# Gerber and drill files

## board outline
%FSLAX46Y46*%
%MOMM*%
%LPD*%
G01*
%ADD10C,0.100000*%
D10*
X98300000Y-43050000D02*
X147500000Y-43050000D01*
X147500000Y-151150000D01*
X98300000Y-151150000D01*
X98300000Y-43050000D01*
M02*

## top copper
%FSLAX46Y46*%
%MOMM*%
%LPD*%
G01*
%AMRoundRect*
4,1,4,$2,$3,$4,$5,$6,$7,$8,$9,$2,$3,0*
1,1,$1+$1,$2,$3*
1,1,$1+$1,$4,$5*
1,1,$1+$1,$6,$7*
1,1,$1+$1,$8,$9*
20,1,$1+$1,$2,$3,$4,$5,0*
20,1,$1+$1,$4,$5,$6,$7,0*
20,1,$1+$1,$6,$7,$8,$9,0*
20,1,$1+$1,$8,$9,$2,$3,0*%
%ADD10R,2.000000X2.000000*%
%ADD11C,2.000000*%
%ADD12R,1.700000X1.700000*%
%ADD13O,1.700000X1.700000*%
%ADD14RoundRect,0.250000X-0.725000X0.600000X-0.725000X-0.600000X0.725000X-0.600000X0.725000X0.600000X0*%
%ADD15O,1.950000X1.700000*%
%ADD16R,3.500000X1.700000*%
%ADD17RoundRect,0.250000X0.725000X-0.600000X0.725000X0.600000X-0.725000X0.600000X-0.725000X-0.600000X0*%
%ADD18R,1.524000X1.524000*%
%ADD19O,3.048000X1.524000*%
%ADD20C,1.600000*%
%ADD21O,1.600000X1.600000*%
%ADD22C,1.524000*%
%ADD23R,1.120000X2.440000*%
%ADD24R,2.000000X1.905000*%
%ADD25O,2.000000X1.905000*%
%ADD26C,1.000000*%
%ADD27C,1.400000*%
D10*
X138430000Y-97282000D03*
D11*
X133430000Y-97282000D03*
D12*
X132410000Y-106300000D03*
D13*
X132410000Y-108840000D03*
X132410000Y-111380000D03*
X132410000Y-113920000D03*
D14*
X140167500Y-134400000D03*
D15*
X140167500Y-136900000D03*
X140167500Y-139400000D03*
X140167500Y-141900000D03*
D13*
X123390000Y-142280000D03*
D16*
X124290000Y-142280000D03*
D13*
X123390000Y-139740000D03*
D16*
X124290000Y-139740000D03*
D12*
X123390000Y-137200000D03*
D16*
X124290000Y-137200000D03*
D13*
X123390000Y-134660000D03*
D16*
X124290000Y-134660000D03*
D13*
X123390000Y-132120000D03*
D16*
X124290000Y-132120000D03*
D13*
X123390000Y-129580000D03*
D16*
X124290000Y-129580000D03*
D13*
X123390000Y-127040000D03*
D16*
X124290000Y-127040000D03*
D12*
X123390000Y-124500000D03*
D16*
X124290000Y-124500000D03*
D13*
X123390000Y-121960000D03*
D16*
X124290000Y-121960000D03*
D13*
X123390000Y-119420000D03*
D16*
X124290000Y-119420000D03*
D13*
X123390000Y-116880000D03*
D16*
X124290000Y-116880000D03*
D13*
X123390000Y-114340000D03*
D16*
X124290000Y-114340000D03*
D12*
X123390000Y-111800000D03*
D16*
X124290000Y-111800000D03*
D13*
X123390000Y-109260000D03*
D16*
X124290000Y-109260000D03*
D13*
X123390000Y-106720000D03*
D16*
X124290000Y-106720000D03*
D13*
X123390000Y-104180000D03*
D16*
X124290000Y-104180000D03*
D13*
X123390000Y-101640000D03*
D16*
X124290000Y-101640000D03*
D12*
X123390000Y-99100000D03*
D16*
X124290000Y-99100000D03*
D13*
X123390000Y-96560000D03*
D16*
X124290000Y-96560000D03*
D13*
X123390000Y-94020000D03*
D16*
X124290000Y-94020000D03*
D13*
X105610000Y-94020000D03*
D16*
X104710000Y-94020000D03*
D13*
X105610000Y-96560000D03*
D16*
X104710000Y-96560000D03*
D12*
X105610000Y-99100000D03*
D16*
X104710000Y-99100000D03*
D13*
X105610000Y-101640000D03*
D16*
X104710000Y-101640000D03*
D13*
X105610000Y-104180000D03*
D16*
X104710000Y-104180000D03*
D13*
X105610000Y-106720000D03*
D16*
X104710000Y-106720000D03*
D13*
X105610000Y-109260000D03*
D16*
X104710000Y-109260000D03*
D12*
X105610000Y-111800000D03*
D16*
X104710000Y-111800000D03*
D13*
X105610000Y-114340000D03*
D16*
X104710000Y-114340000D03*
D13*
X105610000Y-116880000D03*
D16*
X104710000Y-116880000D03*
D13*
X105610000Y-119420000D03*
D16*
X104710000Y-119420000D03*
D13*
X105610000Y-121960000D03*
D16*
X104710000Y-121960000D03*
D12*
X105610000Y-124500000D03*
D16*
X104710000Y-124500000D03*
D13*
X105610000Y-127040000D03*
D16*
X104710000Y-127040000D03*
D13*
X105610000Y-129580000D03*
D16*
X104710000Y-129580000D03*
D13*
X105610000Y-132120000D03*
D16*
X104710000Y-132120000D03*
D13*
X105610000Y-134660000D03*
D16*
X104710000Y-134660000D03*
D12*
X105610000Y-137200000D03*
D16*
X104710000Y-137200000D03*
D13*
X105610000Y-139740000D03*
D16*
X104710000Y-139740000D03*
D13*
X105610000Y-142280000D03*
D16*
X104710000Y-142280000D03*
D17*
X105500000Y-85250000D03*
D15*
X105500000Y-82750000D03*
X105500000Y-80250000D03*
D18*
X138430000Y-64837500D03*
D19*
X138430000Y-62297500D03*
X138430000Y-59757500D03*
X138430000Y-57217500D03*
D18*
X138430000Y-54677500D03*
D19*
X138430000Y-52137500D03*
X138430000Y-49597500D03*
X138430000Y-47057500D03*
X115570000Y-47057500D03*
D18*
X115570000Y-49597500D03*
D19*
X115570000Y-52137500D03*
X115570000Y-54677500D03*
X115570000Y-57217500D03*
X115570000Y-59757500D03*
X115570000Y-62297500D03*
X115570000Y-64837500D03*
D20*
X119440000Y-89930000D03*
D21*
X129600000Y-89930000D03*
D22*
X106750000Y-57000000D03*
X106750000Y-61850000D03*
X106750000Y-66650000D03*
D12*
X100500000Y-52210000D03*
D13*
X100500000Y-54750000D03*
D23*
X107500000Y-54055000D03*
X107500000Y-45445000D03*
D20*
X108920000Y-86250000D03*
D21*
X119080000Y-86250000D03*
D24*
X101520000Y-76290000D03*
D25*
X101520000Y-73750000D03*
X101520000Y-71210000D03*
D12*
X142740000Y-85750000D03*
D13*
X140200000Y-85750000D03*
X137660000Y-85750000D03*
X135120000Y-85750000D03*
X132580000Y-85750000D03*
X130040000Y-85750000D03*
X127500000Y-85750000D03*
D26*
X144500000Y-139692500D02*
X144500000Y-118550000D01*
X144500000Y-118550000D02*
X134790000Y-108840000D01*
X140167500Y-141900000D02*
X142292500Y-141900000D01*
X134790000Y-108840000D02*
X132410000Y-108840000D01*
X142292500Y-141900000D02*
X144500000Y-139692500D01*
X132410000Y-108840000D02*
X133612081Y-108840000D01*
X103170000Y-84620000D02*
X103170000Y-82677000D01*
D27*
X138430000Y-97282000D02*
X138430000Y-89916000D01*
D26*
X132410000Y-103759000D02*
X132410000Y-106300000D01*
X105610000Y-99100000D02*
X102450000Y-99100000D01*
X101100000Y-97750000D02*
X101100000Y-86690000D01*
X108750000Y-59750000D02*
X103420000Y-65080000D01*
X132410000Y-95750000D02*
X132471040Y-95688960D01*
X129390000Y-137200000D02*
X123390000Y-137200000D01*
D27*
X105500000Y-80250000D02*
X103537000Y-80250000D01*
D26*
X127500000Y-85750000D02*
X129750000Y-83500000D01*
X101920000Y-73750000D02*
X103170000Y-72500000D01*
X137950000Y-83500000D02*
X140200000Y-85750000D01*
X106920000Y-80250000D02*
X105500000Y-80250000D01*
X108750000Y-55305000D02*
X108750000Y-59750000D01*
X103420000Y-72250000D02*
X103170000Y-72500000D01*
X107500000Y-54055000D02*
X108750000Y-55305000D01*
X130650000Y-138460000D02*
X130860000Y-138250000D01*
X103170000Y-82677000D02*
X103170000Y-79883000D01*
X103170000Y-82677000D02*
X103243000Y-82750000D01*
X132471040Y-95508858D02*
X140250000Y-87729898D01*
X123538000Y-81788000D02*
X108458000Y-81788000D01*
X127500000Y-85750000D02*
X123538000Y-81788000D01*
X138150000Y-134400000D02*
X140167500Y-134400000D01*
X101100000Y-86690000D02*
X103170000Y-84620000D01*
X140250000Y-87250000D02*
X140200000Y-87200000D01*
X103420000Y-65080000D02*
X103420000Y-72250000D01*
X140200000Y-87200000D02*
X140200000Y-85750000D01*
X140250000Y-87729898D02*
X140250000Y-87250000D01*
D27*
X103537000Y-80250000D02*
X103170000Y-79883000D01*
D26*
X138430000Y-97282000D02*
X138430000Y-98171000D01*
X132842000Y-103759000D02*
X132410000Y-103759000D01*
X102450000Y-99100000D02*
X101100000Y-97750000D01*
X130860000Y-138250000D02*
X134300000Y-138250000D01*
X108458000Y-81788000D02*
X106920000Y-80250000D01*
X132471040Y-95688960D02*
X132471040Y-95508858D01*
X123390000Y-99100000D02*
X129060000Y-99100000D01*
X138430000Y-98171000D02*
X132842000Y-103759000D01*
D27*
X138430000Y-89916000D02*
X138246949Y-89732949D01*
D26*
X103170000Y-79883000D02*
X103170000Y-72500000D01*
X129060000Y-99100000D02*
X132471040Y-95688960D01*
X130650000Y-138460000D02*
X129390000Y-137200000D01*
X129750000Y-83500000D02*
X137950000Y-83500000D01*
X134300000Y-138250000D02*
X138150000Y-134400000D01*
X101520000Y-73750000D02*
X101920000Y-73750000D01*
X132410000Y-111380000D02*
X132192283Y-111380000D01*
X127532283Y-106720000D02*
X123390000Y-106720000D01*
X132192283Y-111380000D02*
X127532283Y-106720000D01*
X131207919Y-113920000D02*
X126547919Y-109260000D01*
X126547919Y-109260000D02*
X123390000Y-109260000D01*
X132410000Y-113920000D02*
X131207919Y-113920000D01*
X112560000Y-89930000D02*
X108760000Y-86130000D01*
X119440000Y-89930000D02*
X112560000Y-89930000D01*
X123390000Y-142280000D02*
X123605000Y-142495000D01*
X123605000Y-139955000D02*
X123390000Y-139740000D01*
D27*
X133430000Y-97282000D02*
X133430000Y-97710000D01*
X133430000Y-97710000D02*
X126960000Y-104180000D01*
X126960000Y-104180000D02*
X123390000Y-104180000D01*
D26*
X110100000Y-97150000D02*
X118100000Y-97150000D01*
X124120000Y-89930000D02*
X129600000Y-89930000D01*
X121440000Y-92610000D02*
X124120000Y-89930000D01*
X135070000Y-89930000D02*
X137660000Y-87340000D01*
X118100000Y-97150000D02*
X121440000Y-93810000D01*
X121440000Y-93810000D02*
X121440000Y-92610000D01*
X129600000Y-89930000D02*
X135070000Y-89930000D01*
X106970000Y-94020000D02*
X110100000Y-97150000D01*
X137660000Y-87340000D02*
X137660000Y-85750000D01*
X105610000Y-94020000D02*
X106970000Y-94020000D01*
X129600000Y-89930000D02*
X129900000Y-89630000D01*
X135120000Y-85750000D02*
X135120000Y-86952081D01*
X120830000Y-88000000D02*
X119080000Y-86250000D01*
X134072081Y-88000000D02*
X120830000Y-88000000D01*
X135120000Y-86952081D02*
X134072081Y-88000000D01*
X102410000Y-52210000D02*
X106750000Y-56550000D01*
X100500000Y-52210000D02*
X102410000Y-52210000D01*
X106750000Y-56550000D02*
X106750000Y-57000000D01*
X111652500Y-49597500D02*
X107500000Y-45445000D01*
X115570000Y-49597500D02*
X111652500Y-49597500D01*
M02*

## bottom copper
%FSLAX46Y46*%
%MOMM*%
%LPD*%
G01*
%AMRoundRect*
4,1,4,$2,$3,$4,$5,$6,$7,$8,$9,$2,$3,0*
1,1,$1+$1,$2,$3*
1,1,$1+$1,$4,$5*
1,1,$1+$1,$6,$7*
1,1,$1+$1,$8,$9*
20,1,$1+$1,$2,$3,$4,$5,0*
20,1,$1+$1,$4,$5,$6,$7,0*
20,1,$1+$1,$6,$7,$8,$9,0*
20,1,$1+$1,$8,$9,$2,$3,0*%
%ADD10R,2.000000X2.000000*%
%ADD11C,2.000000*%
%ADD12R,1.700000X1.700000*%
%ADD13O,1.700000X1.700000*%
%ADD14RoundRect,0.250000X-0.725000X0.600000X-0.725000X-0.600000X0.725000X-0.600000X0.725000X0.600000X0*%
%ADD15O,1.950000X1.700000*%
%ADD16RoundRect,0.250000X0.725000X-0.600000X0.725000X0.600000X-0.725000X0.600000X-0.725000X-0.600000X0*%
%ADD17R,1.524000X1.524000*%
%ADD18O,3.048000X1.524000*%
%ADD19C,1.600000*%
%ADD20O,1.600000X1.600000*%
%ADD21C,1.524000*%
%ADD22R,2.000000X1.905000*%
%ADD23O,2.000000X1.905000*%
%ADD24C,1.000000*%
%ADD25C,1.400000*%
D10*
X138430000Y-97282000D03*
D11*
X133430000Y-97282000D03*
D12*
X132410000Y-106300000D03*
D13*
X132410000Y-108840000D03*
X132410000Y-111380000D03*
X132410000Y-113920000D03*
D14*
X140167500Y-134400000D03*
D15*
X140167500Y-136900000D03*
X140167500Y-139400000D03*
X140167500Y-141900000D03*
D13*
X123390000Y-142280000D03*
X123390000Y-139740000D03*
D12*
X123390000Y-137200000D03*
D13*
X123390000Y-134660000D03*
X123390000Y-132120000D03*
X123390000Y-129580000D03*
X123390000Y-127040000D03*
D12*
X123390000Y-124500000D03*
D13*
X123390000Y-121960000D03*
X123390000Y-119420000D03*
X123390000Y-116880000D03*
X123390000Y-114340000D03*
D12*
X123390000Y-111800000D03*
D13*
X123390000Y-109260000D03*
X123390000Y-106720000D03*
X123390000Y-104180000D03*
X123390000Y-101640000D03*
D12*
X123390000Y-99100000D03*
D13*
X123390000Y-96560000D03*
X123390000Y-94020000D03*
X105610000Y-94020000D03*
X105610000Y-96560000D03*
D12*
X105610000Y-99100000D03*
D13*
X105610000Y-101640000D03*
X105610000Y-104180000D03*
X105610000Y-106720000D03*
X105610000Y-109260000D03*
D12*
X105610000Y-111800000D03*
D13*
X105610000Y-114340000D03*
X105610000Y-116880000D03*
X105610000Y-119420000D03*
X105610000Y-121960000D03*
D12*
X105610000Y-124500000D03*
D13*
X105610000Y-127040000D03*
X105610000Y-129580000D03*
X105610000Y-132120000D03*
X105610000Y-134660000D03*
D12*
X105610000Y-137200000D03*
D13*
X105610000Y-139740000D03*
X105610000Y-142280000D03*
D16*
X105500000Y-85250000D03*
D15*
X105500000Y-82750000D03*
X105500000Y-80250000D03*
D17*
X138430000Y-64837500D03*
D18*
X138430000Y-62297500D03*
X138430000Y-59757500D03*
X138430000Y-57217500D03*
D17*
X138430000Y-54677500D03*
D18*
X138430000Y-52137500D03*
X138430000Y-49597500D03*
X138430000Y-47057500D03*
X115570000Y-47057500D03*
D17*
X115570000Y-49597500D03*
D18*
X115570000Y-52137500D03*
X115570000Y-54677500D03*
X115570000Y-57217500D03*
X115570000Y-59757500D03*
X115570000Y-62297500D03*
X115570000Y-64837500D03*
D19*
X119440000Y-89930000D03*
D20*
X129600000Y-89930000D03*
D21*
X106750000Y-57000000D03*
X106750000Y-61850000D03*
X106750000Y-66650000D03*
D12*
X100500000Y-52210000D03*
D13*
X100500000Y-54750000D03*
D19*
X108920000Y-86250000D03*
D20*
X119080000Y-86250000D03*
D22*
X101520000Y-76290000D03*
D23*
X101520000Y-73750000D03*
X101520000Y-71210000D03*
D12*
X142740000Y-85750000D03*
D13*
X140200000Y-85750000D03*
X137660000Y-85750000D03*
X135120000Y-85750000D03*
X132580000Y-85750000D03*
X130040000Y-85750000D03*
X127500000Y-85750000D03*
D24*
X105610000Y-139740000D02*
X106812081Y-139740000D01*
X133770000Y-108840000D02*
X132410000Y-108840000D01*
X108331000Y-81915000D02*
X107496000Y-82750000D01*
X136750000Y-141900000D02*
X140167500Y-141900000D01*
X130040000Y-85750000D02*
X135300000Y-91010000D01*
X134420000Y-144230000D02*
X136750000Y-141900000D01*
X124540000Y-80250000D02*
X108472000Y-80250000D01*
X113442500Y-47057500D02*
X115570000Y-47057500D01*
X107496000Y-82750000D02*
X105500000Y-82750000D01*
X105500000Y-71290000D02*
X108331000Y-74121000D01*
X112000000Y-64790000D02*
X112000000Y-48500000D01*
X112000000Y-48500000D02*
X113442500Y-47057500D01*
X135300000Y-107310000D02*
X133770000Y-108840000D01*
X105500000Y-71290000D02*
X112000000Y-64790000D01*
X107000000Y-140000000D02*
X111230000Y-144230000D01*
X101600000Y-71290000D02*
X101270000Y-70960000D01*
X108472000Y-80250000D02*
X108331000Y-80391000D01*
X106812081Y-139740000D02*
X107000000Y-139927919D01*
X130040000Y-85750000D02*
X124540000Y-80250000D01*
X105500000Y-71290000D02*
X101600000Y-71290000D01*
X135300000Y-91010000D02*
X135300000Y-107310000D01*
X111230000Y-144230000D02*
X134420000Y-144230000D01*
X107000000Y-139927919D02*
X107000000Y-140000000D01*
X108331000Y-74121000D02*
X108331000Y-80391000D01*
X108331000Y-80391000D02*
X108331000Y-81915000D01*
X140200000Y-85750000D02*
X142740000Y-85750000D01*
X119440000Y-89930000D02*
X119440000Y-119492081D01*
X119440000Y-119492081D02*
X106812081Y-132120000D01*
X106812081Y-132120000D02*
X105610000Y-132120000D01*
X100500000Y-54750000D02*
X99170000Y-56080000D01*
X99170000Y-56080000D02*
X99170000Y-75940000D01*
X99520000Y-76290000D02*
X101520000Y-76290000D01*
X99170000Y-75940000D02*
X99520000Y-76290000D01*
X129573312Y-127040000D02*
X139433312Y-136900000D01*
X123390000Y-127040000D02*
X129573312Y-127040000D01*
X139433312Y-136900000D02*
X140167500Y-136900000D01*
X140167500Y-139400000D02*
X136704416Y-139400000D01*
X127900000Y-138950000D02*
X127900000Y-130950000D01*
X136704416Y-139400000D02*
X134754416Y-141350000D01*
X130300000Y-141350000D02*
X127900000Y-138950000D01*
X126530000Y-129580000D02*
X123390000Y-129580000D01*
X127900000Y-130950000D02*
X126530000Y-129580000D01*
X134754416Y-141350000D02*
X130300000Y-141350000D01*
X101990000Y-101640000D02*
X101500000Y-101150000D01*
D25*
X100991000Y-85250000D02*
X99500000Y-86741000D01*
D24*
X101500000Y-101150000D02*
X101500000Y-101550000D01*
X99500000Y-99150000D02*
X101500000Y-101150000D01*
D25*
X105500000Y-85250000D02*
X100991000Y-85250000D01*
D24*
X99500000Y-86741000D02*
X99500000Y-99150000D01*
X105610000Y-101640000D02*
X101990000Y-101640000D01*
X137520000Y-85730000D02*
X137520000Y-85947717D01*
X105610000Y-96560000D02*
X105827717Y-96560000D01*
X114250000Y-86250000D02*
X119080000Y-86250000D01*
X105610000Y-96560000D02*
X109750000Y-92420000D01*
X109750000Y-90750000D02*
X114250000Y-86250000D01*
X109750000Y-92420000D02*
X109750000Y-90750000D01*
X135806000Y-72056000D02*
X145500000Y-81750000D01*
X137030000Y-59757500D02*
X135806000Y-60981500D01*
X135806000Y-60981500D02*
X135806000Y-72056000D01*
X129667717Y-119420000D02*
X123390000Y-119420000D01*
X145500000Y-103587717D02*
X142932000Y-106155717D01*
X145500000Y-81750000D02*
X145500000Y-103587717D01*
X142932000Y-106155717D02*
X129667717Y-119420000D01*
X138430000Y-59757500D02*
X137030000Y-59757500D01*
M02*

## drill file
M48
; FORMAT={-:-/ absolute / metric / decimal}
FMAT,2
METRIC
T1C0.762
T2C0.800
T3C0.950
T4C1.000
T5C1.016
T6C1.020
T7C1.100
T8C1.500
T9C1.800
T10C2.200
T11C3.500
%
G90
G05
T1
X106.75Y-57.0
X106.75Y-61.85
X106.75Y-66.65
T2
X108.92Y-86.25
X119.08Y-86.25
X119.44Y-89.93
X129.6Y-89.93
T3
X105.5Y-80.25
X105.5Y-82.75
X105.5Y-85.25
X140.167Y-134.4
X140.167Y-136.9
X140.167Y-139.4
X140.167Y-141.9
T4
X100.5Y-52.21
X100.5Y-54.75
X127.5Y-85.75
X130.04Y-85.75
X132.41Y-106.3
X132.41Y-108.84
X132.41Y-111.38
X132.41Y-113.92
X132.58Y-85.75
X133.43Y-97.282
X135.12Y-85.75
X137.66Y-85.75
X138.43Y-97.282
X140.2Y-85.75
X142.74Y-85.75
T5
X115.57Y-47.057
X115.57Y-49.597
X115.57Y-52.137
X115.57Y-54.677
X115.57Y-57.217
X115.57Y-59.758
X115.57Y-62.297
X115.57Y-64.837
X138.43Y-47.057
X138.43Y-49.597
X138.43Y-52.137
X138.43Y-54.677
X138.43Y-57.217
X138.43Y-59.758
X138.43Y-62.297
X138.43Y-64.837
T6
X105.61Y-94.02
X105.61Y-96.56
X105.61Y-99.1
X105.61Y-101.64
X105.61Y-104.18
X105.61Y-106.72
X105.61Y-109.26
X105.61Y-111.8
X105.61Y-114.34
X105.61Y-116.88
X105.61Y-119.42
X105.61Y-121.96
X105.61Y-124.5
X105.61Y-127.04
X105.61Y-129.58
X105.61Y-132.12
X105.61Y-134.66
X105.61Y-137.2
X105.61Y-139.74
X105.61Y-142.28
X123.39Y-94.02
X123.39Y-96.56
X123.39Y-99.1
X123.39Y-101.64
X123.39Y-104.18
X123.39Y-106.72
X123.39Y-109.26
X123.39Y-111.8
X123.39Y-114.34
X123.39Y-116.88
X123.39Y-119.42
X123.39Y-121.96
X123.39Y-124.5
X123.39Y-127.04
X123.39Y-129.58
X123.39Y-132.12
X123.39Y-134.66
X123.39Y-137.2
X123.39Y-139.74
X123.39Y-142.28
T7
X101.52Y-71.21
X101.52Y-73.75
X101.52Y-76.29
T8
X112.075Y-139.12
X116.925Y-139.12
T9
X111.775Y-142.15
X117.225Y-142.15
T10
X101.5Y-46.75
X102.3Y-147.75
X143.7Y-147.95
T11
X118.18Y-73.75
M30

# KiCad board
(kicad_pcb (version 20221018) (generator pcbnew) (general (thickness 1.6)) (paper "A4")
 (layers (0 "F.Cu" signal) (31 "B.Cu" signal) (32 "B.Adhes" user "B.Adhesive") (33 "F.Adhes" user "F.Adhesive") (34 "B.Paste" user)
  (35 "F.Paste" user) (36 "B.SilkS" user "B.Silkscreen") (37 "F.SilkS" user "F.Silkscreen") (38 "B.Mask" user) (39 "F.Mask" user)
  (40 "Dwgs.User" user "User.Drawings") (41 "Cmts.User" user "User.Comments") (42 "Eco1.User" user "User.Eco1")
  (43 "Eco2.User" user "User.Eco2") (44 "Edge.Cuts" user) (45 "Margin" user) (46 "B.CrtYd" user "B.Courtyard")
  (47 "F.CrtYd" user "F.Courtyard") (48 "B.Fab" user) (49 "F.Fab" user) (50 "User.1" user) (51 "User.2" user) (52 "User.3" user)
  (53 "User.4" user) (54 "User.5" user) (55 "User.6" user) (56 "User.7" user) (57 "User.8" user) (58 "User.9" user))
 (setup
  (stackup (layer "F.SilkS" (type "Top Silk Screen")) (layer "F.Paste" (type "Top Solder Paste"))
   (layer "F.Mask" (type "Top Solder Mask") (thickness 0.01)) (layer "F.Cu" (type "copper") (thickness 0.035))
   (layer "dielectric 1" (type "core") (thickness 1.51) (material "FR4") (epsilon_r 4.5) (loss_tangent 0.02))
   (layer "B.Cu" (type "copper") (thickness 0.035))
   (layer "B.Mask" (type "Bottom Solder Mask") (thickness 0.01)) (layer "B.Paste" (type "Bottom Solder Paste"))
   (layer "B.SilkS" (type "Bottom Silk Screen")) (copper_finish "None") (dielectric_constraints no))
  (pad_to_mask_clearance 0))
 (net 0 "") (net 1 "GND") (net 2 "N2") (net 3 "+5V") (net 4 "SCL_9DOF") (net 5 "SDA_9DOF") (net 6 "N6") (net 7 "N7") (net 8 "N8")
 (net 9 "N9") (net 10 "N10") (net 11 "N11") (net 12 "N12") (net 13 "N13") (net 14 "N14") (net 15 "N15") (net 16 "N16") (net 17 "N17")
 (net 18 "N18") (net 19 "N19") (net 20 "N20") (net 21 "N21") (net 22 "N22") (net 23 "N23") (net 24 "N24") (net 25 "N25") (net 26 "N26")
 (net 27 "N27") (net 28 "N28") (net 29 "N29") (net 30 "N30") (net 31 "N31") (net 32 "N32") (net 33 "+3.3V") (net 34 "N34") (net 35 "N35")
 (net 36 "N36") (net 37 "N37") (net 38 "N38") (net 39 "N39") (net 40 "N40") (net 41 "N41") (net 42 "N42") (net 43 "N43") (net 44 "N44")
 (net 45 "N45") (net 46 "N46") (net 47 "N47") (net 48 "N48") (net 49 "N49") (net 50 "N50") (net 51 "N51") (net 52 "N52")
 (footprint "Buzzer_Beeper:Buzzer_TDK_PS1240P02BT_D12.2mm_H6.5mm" (layer "F.Cu") (at 138.43 97.282 180)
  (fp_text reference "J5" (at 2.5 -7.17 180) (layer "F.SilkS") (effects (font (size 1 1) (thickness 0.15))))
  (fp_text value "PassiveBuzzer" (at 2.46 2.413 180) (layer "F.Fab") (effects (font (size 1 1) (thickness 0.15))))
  (pad "1" thru_hole rect (at 0 0 180) (size 2 2) (drill 1) (layers "*.Cu" "*.Mask") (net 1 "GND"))
  (pad "2" thru_hole circle (at 5 0 180) (size 2 2) (drill 1) (layers "*.Cu" "*.Mask") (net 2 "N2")))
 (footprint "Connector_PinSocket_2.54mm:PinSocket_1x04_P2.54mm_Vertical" (layer "F.Cu") (at 132.41 106.3)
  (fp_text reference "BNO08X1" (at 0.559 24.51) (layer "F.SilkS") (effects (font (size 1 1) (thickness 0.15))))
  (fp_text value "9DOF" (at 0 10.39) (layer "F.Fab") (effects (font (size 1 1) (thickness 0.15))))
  (pad "1" thru_hole rect (at 0 0) (size 1.7 1.7) (drill 1) (layers "*.Cu" "*.Mask") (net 1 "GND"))
  (pad "2" thru_hole oval (at 0 2.54) (size 1.7 1.7) (drill 1) (layers "*.Cu" "*.Mask") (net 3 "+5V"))
  (pad "3" thru_hole oval (at 0 5.08) (size 1.7 1.7) (drill 1) (layers "*.Cu" "*.Mask") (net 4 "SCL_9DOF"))
  (pad "4" thru_hole oval (at 0 7.62) (size 1.7 1.7) (drill 1) (layers "*.Cu" "*.Mask") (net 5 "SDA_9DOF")))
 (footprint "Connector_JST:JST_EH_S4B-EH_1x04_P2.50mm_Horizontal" (layer "F.Cu") (at 140.1675 134.4 -90)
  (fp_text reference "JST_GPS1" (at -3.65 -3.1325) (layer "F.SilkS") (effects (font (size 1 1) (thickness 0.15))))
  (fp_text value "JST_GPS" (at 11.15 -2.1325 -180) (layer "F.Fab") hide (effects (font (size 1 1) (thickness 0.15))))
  (pad "1" thru_hole roundrect (at 0 0 270) (size 1.7 1.95) (drill 0.95) (layers "*.Cu" "*.Mask") (roundrect_rratio 0.1470588235)
   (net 1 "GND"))
  (pad "2" thru_hole oval (at 2.5 0 270) (size 1.7 1.95) (drill 0.95) (layers "*.Cu" "*.Mask") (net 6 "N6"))
  (pad "3" thru_hole oval (at 5 0 270) (size 1.7 1.95) (drill 0.95) (layers "*.Cu" "*.Mask") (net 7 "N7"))
  (pad "4" thru_hole oval (at 7.5 0 270) (size 1.7 1.95) (drill 0.95) (layers "*.Cu" "*.Mask") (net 3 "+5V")))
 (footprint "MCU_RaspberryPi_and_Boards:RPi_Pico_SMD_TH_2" (layer "F.Cu") (at 114.5 118.15 180)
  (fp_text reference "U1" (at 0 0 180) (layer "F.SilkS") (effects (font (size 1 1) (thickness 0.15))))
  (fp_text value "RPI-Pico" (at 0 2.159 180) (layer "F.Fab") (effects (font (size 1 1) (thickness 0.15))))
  (pad "" np_thru_hole oval (at -2.725 -24 180) (size 1.8 1.8) (drill 1.8) (layers "*.Cu" "*.Mask"))
  (pad "" np_thru_hole oval (at -2.425 -20.97 180) (size 1.5 1.5) (drill 1.5) (layers "*.Cu" "*.Mask"))
  (pad "" np_thru_hole oval (at 2.425 -20.97 180) (size 1.5 1.5) (drill 1.5) (layers "*.Cu" "*.Mask"))
  (pad "" np_thru_hole oval (at 2.725 -24 180) (size 1.8 1.8) (drill 1.8) (layers "*.Cu" "*.Mask"))
  (pad "1" thru_hole oval (at -8.89 -24.13 180) (size 1.7 1.7) (drill 1.02) (layers "*.Cu" "*.Mask") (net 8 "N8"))
  (pad "1" smd rect (at -8.89 -24.13 180) (size 3.5 1.7) (drill (offset -0.9 0)) (layers "F.Cu" "F.Mask") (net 8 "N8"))
  (pad "2" thru_hole oval (at -8.89 -21.59 180) (size 1.7 1.7) (drill 1.02) (layers "*.Cu" "*.Mask") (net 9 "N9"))
  (pad "2" smd rect (at -8.89 -21.59 180) (size 3.5 1.7) (drill (offset -0.9 0)) (layers "F.Cu" "F.Mask") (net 9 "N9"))
  (pad "3" thru_hole rect (at -8.89 -19.05 180) (size 1.7 1.7) (drill 1.02) (layers "*.Cu" "*.Mask") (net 1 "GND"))
  (pad "3" smd rect (at -8.89 -19.05 180) (size 3.5 1.7) (drill (offset -0.9 0)) (layers "F.Cu" "F.Mask") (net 1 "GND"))
  (pad "4" thru_hole oval (at -8.89 -16.51 180) (size 1.7 1.7) (drill 1.02) (layers "*.Cu" "*.Mask") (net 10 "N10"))
  (pad "4" smd rect (at -8.89 -16.51 180) (size 3.5 1.7) (drill (offset -0.9 0)) (layers "F.Cu" "F.Mask") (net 10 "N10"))
  (pad "5" thru_hole oval (at -8.89 -13.97 180) (size 1.7 1.7) (drill 1.02) (layers "*.Cu" "*.Mask") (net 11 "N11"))
  (pad "5" smd rect (at -8.89 -13.97 180) (size 3.5 1.7) (drill (offset -0.9 0)) (layers "F.Cu" "F.Mask") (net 11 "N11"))
  (pad "6" thru_hole oval (at -8.89 -11.43 180) (size 1.7 1.7) (drill 1.02) (layers "*.Cu" "*.Mask") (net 7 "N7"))
  (pad "6" smd rect (at -8.89 -11.43 180) (size 3.5 1.7) (drill (offset -0.9 0)) (layers "F.Cu" "F.Mask") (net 7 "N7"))
  (pad "7" thru_hole oval (at -8.89 -8.89 180) (size 1.7 1.7) (drill 1.02) (layers "*.Cu" "*.Mask") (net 6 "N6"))
  (pad "7" smd rect (at -8.89 -8.89 180) (size 3.5 1.7) (drill (offset -0.9 0)) (layers "F.Cu" "F.Mask") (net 6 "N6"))
  (pad "8" thru_hole rect (at -8.89 -6.35 180) (size 1.7 1.7) (drill 1.02) (layers "*.Cu" "*.Mask") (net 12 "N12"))
  (pad "8" smd rect (at -8.89 -6.35 180) (size 3.5 1.7) (drill (offset -0.9 0)) (layers "F.Cu" "F.Mask") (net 12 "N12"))
  (pad "9" thru_hole oval (at -8.89 -3.81 180) (size 1.7 1.7) (drill 1.02) (layers "*.Cu" "*.Mask") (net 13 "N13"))
  (pad "9" smd rect (at -8.89 -3.81 180) (size 3.5 1.7) (drill (offset -0.9 0)) (layers "F.Cu" "F.Mask") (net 13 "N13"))
  (pad "10" thru_hole oval (at -8.89 -1.27 180) (size 1.7 1.7) (drill 1.02) (layers "*.Cu" "*.Mask") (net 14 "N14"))
  (pad "10" smd rect (at -8.89 -1.27 180) (size 3.5 1.7) (drill (offset -0.9 0)) (layers "F.Cu" "F.Mask") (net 14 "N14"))
  (pad "11" thru_hole oval (at -8.89 1.27 180) (size 1.7 1.7) (drill 1.02) (layers "*.Cu" "*.Mask") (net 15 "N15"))
  (pad "11" smd rect (at -8.89 1.27 180) (size 3.5 1.7) (drill (offset -0.9 0)) (layers "F.Cu" "F.Mask") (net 15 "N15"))
  (pad "12" thru_hole oval (at -8.89 3.81 180) (size 1.7 1.7) (drill 1.02) (layers "*.Cu" "*.Mask") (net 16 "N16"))
  (pad "12" smd rect (at -8.89 3.81 180) (size 3.5 1.7) (drill (offset -0.9 0)) (layers "F.Cu" "F.Mask") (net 16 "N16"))
  (pad "13" thru_hole rect (at -8.89 6.35 180) (size 1.7 1.7) (drill 1.02) (layers "*.Cu" "*.Mask") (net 1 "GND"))
  (pad "13" smd rect (at -8.89 6.35 180) (size 3.5 1.7) (drill (offset -0.9 0)) (layers "F.Cu" "F.Mask") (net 1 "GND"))
  (pad "14" thru_hole oval (at -8.89 8.89 180) (size 1.7 1.7) (drill 1.02) (layers "*.Cu" "*.Mask") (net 5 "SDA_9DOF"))
  (pad "14" smd rect (at -8.89 8.89 180) (size 3.5 1.7) (drill (offset -0.9 0)) (layers "F.Cu" "F.Mask") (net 5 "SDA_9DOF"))
  (pad "15" thru_hole oval (at -8.89 11.43 180) (size 1.7 1.7) (drill 1.02) (layers "*.Cu" "*.Mask") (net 4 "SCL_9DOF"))
  (pad "15" smd rect (at -8.89 11.43 180) (size 3.5 1.7) (drill (offset -0.9 0)) (layers "F.Cu" "F.Mask") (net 4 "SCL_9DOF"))
  (pad "16" thru_hole oval (at -8.89 13.97 180) (size 1.7 1.7) (drill 1.02) (layers "*.Cu" "*.Mask") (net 2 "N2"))
  (pad "16" smd rect (at -8.89 13.97 180) (size 3.5 1.7) (drill (offset -0.9 0)) (layers "F.Cu" "F.Mask") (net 2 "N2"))
  (pad "17" thru_hole oval (at -8.89 16.51 180) (size 1.7 1.7) (drill 1.02) (layers "*.Cu" "*.Mask") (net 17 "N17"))
  (pad "17" smd rect (at -8.89 16.51 180) (size 3.5 1.7) (drill (offset -0.9 0)) (layers "F.Cu" "F.Mask") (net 17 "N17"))
  (pad "18" thru_hole rect (at -8.89 19.05 180) (size 1.7 1.7) (drill 1.02) (layers "*.Cu" "*.Mask") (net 1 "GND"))
  (pad "18" smd rect (at -8.89 19.05 180) (size 3.5 1.7) (drill (offset -0.9 0)) (layers "F.Cu" "F.Mask") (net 1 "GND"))
  (pad "19" thru_hole oval (at -8.89 21.59 180) (size 1.7 1.7) (drill 1.02) (layers "*.Cu" "*.Mask") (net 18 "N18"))
  (pad "19" smd rect (at -8.89 21.59 180) (size 3.5 1.7) (drill (offset -0.9 0)) (layers "F.Cu" "F.Mask") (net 18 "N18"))
  (pad "20" thru_hole oval (at -8.89 24.13 180) (size 1.7 1.7) (drill 1.02) (layers "*.Cu" "*.Mask") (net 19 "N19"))
  (pad "20" smd rect (at -8.89 24.13 180) (size 3.5 1.7) (drill (offset -0.9 0)) (layers "F.Cu" "F.Mask") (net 19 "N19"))
  (pad "21" thru_hole oval (at 8.89 24.13 180) (size 1.7 1.7) (drill 1.02) (layers "*.Cu" "*.Mask") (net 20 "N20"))
  (pad "21" smd rect (at 8.89 24.13 180) (size 3.5 1.7) (drill (offset 0.9 0)) (layers "F.Cu" "F.Mask") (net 20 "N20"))
  (pad "22" thru_hole oval (at 8.89 21.59 180) (size 1.7 1.7) (drill 1.02) (layers "*.Cu" "*.Mask") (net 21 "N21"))
  (pad "22" smd rect (at 8.89 21.59 180) (size 3.5 1.7) (drill (offset 0.9 0)) (layers "F.Cu" "F.Mask") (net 21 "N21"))
  (pad "23" thru_hole rect (at 8.89 19.05 180) (size 1.7 1.7) (drill 1.02) (layers "*.Cu" "*.Mask") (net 1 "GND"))
  (pad "23" smd rect (at 8.89 19.05 180) (size 3.5 1.7) (drill (offset 0.9 0)) (layers "F.Cu" "F.Mask") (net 1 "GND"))
  (pad "24" thru_hole oval (at 8.89 16.51 180) (size 1.7 1.7) (drill 1.02) (layers "*.Cu" "*.Mask") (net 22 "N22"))
  (pad "24" smd rect (at 8.89 16.51 180) (size 3.5 1.7) (drill (offset 0.9 0)) (layers "F.Cu" "F.Mask") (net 22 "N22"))
  (pad "25" thru_hole oval (at 8.89 13.97 180) (size 1.7 1.7) (drill 1.02) (layers "*.Cu" "*.Mask") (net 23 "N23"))
  (pad "25" smd rect (at 8.89 13.97 180) (size 3.5 1.7) (drill (offset 0.9 0)) (layers "F.Cu" "F.Mask") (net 23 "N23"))
  (pad "26" thru_hole oval (at 8.89 11.43 180) (size 1.7 1.7) (drill 1.02) (layers "*.Cu" "*.Mask") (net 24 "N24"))
  (pad "26" smd rect (at 8.89 11.43 180) (size 3.5 1.7) (drill (offset 0.9 0)) (layers "F.Cu" "F.Mask") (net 24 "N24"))
  (pad "27" thru_hole oval (at 8.89 8.89 180) (size 1.7 1.7) (drill 1.02) (layers "*.Cu" "*.Mask") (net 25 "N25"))
  (pad "27" smd rect (at 8.89 8.89 180) (size 3.5 1.7) (drill (offset 0.9 0)) (layers "F.Cu" "F.Mask") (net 25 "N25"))
  (pad "28" thru_hole rect (at 8.89 6.35 180) (size 1.7 1.7) (drill 1.02) (layers "*.Cu" "*.Mask") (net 1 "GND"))
  (pad "28" smd rect (at 8.89 6.35 180) (size 3.5 1.7) (drill (offset 0.9 0)) (layers "F.Cu" "F.Mask") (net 1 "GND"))
  (pad "29" thru_hole oval (at 8.89 3.81 180) (size 1.7 1.7) (drill 1.02) (layers "*.Cu" "*.Mask") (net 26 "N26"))
  (pad "29" smd rect (at 8.89 3.81 180) (size 3.5 1.7) (drill (offset 0.9 0)) (layers "F.Cu" "F.Mask") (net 26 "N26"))
  (pad "30" thru_hole oval (at 8.89 1.27 180) (size 1.7 1.7) (drill 1.02) (layers "*.Cu" "*.Mask") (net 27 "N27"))
  (pad "30" smd rect (at 8.89 1.27 180) (size 3.5 1.7) (drill (offset 0.9 0)) (layers "F.Cu" "F.Mask") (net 27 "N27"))
  (pad "31" thru_hole oval (at 8.89 -1.27 180) (size 1.7 1.7) (drill 1.02) (layers "*.Cu" "*.Mask") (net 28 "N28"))
  (pad "31" smd rect (at 8.89 -1.27 180) (size 3.5 1.7) (drill (offset 0.9 0)) (layers "F.Cu" "F.Mask") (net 28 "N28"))
  (pad "32" thru_hole oval (at 8.89 -3.81 180) (size 1.7 1.7) (drill 1.02) (layers "*.Cu" "*.Mask") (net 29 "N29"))
  (pad "32" smd rect (at 8.89 -3.81 180) (size 3.5 1.7) (drill (offset 0.9 0)) (layers "F.Cu" "F.Mask") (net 29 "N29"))
  (pad "33" thru_hole rect (at 8.89 -6.35 180) (size 1.7 1.7) (drill 1.02) (layers "*.Cu" "*.Mask") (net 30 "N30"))
  (pad "33" smd rect (at 8.89 -6.35 180) (size 3.5 1.7) (drill (offset 0.9 0)) (layers "F.Cu" "F.Mask") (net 30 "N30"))
  (pad "34" thru_hole oval (at 8.89 -8.89 180) (size 1.7 1.7) (drill 1.02) (layers "*.Cu" "*.Mask") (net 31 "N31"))
  (pad "34" smd rect (at 8.89 -8.89 180) (size 3.5 1.7) (drill (offset 0.9 0)) (layers "F.Cu" "F.Mask") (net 31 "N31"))
  (pad "35" thru_hole oval (at 8.89 -11.43 180) (size 1.7 1.7) (drill 1.02) (layers "*.Cu" "*.Mask") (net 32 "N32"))
  (pad "35" smd rect (at 8.89 -11.43 180) (size 3.5 1.7) (drill (offset 0.9 0)) (layers "F.Cu" "F.Mask") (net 32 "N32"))
  (pad "36" thru_hole oval (at 8.89 -13.97 180) (size 1.7 1.7) (drill 1.02) (layers "*.Cu" "*.Mask") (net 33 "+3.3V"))
  (pad "36" smd rect (at 8.89 -13.97 180) (size 3.5 1.7) (drill (offset 0.9 0)) (layers "F.Cu" "F.Mask") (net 33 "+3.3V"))
  (pad "37" thru_hole oval (at 8.89 -16.51 180) (size 1.7 1.7) (drill 1.02) (layers "*.Cu" "*.Mask") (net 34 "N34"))
  (pad "37" smd rect (at 8.89 -16.51 180) (size 3.5 1.7) (drill (offset 0.9 0)) (layers "F.Cu" "F.Mask") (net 34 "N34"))
  (pad "38" thru_hole rect (at 8.89 -19.05 180) (size 1.7 1.7) (drill 1.02) (layers "*.Cu" "*.Mask") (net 1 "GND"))
  (pad "38" smd rect (at 8.89 -19.05 180) (size 3.5 1.7) (drill (offset 0.9 0)) (layers "F.Cu" "F.Mask") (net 1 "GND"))
  (pad "39" thru_hole oval (at 8.89 -21.59 180) (size 1.7 1.7) (drill 1.02) (layers "*.Cu" "*.Mask") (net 3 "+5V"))
  (pad "39" smd rect (at 8.89 -21.59 180) (size 3.5 1.7) (drill (offset 0.9 0)) (layers "F.Cu" "F.Mask") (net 3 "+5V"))
  (pad "40" thru_hole oval (at 8.89 -24.13 180) (size 1.7 1.7) (drill 1.02) (layers "*.Cu" "*.Mask") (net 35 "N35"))
  (pad "40" smd rect (at 8.89 -24.13 180) (size 3.5 1.7) (drill (offset 0.9 0)) (layers "F.Cu" "F.Mask") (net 35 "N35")))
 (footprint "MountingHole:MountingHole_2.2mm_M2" (layer "F.Cu") (at 102.3 147.75)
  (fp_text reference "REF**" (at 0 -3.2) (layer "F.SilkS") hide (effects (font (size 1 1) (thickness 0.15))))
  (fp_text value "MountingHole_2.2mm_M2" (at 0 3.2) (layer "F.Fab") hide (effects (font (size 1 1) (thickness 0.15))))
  (pad "" np_thru_hole circle (at 0 0) (size 2.2 2.2) (drill 2.2) (layers "F&B.Cu" "*.Mask")))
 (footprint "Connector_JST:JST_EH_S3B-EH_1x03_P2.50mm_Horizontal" (layer "F.Cu") (at 105.5 85.25 90)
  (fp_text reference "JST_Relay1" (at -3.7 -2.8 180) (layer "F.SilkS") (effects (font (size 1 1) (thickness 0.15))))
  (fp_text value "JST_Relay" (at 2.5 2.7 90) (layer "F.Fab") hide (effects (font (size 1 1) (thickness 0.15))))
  (pad "1" thru_hole roundrect (at 0 0 90) (size 1.7 1.95) (drill 0.95) (layers "*.Cu" "*.Mask") (roundrect_rratio 0.1470588235)
   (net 22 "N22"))
  (pad "2" thru_hole oval (at 2.5 0 90) (size 1.7 1.95) (drill 0.95) (layers "*.Cu" "*.Mask") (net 3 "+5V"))
  (pad "3" thru_hole oval (at 5 0 90) (size 1.7 1.95) (drill 0.95) (layers "*.Cu" "*.Mask") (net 1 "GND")))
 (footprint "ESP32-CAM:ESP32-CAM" (layer "F.Cu") (at 127 57.2175 180)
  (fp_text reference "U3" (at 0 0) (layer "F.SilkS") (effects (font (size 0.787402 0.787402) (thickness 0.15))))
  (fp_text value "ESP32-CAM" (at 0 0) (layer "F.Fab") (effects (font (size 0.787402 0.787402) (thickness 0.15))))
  (pad "P$1" thru_hole rect (at -11.43 -7.62 180) (size 1.524 1.524) (drill 1.016) (layers "*.Cu" "*.Mask") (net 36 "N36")
   (solder_mask_margin 0.102))
  (pad "P$2" thru_hole oval (at -11.43 -5.08 180) (size 3.048 1.524) (drill 1.016) (layers "*.Cu" "*.Mask") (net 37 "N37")
   (solder_mask_margin 0.102))
  (pad "P$3" thru_hole oval (at -11.43 -2.54 180) (size 3.048 1.524) (drill 1.016) (layers "*.Cu" "*.Mask") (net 14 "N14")
   (solder_mask_margin 0.102))
  (pad "P$4" thru_hole oval (at -11.43 0 180) (size 3.048 1.524) (drill 1.016) (layers "*.Cu" "*.Mask") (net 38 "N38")
   (solder_mask_margin 0.102))
  (pad "P$5" thru_hole rect (at -11.43 2.54 180) (size 1.524 1.524) (drill 1.016) (layers "*.Cu" "*.Mask") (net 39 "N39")
   (solder_mask_margin 0.102))
  (pad "P$6" thru_hole oval (at -11.43 5.08 180) (size 3.048 1.524) (drill 1.016) (layers "*.Cu" "*.Mask") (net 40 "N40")
   (solder_mask_margin 0.102))
  (pad "P$7" thru_hole oval (at -11.43 7.62 180) (size 3.048 1.524) (drill 1.016) (layers "*.Cu" "*.Mask") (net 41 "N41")
   (solder_mask_margin 0.102))
  (pad "P$8" thru_hole oval (at -11.43 10.16 180) (size 3.048 1.524) (drill 1.016) (layers "*.Cu" "*.Mask") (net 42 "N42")
   (solder_mask_margin 0.102))
  (pad "P$9" thru_hole oval (at 11.43 10.16 180) (size 3.048 1.524) (drill 1.016) (layers "*.Cu" "*.Mask") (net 3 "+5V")
   (solder_mask_margin 0.102))
  (pad "P$10" thru_hole rect (at 11.43 7.62 180) (size 1.524 1.524) (drill 1.016) (layers "*.Cu" "*.Mask") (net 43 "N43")
   (solder_mask_margin 0.102))
  (pad "P$11" thru_hole oval (at 11.43 5.08 180) (size 3.048 1.524) (drill 1.016) (layers "*.Cu" "*.Mask") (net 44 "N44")
   (solder_mask_margin 0.102))
  (pad "P$12" thru_hole oval (at 11.43 2.54 180) (size 3.048 1.524) (drill 1.016) (layers "*.Cu" "*.Mask") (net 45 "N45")
   (solder_mask_margin 0.102))
  (pad "P$13" thru_hole oval (at 11.43 0 180) (size 3.048 1.524) (drill 1.016) (layers "*.Cu" "*.Mask") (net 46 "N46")
   (solder_mask_margin 0.102))
  (pad "P$14" thru_hole oval (at 11.43 -2.54 180) (size 3.048 1.524) (drill 1.016) (layers "*.Cu" "*.Mask") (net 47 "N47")
   (solder_mask_margin 0.102))
  (pad "P$15" thru_hole oval (at 11.43 -5.08 180) (size 3.048 1.524) (drill 1.016) (layers "*.Cu" "*.Mask") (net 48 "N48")
   (solder_mask_margin 0.102))
  (pad "P$16" thru_hole oval (at 11.43 -7.62 180) (size 3.048 1.524) (drill 1.016) (layers "*.Cu" "*.Mask") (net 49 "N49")
   (solder_mask_margin 0.102)))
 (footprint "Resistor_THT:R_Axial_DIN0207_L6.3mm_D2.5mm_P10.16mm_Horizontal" (layer "F.Cu") (at 119.44 89.93)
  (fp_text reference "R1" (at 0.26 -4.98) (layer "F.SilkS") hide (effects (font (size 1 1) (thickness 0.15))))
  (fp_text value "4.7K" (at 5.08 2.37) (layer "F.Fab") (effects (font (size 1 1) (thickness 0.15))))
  (pad "1" thru_hole circle (at 0 0) (size 1.6 1.6) (drill 0.8) (layers "*.Cu" "*.Mask") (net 33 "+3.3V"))
  (pad "2" thru_hole oval (at 10.16 0) (size 1.6 1.6) (drill 0.8) (layers "*.Cu" "*.Mask") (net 20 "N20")))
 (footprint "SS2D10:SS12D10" (layer "F.Cu") (at 108.35 71.25)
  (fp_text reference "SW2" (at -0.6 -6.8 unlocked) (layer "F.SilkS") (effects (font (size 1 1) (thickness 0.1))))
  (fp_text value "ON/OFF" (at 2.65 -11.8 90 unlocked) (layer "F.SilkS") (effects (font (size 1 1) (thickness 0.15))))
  (pad "1" thru_hole circle (at -1.6 -14.25) (size 1.524 1.524) (drill 0.762) (layers "*.Cu" "*.Mask") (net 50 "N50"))
  (pad "2" thru_hole circle (at -1.6 -9.4) (size 1.524 1.524) (drill 0.762) (layers "*.Cu" "*.Mask") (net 1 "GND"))
  (pad "3" thru_hole circle (at -1.6 -4.6) (size 1.524 1.524) (drill 0.762) (layers "*.Cu" "*.Mask")))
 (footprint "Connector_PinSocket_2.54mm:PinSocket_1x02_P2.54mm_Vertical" (layer "F.Cu") (at 100.5 52.21)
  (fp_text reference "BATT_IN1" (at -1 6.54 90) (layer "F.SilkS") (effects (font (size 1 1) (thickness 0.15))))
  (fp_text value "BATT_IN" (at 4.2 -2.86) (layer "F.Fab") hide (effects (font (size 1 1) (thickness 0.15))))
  (pad "1" thru_hole rect (at 0 0) (size 1.7 1.7) (drill 1) (layers "*.Cu" "*.Mask") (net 50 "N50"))
  (pad "2" thru_hole oval (at 0 2.54) (size 1.7 1.7) (drill 1) (layers "*.Cu" "*.Mask") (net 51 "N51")))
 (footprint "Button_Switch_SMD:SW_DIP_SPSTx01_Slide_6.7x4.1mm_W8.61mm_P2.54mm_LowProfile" (layer "F.Cu") (at 107.5 49.75 90)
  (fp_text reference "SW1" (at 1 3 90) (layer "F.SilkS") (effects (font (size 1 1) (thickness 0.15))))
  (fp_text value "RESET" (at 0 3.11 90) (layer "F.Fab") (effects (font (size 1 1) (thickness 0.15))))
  (pad "1" smd rect (at -4.305 0 90) (size 2.44 1.12) (layers "F.Cu" "F.Paste" "F.Mask") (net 1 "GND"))
  (pad "2" smd rect (at 4.305 0 90) (size 2.44 1.12) (layers "F.Cu" "F.Paste" "F.Mask") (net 43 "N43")))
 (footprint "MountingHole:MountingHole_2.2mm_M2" (layer "F.Cu") (at 101.5 46.75)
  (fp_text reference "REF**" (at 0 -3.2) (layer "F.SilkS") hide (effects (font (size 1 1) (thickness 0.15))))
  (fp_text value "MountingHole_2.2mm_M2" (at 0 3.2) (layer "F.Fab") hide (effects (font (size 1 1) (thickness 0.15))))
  (pad "" np_thru_hole circle (at 0 0) (size 2.2 2.2) (drill 2.2) (layers "F&B.Cu" "*.Mask")))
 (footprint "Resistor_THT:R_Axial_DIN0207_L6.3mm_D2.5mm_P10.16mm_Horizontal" (layer "F.Cu") (at 108.92 86.25)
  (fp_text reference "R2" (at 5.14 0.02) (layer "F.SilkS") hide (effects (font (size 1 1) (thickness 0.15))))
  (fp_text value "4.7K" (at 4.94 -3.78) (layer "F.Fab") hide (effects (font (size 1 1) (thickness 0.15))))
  (pad "1" thru_hole circle (at 0 0) (size 1.6 1.6) (drill 0.8) (layers "*.Cu" "*.Mask") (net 33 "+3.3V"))
  (pad "2" thru_hole oval (at 10.16 0) (size 1.6 1.6) (drill 0.8) (layers "*.Cu" "*.Mask") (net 21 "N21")))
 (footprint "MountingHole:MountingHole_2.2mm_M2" (layer "F.Cu") (at 143.7 147.95)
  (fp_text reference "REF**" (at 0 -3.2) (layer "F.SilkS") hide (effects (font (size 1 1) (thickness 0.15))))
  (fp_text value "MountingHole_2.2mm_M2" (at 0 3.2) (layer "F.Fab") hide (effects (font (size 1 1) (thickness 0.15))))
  (pad "" np_thru_hole circle (at 0 0) (size 2.2 2.2) (drill 2.2) (layers "F&B.Cu" "*.Mask")))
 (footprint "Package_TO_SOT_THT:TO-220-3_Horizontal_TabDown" (layer "B.Cu") (at 101.52 76.29 90)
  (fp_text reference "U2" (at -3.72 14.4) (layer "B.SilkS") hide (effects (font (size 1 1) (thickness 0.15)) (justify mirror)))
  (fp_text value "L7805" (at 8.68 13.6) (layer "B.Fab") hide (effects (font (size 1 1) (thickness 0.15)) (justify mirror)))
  (pad "" np_thru_hole oval (at 2.54 16.66 90) (size 3.5 3.5) (drill 3.5) (layers "*.Cu" "*.Mask"))
  (pad "1" thru_hole rect (at 0 0 90) (size 1.905 2) (drill 1.1) (layers "*.Cu" "*.Mask") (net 51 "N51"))
  (pad "2" thru_hole oval (at 2.54 0 90) (size 1.905 2) (drill 1.1) (layers "*.Cu" "*.Mask") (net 1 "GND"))
  (pad "3" thru_hole oval (at 5.08 0 90) (size 1.905 2) (drill 1.1) (layers "*.Cu" "*.Mask") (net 3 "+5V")))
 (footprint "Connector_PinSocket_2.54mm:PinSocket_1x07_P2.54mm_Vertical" (layer "B.Cu") (at 142.74 85.75 90)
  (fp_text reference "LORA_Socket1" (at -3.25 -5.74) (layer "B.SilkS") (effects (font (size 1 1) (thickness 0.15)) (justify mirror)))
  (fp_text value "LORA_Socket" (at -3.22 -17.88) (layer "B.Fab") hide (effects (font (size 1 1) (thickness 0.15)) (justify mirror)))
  (pad "1" thru_hole rect (at 0 0 90) (size 1.7 1.7) (drill 1) (layers "*.Cu" "*.Mask") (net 1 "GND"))
  (pad "2" thru_hole oval (at 0 -2.54 90) (size 1.7 1.7) (drill 1) (layers "*.Cu" "*.Mask") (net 1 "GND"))
  (pad "3" thru_hole oval (at 0 -5.08 90) (size 1.7 1.7) (drill 1) (layers "*.Cu" "*.Mask") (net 20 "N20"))
  (pad "4" thru_hole oval (at 0 -7.62 90) (size 1.7 1.7) (drill 1) (layers "*.Cu" "*.Mask") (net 21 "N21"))
  (pad "5" thru_hole oval (at 0 -10.16 90) (size 1.7 1.7) (drill 1) (layers "*.Cu" "*.Mask") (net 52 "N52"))
  (pad "6" thru_hole oval (at 0 -12.7 90) (size 1.7 1.7) (drill 1) (layers "*.Cu" "*.Mask") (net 3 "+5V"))
  (pad "7" thru_hole oval (at 0 -15.24 90) (size 1.7 1.7) (drill 1) (layers "*.Cu" "*.Mask") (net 1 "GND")))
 (gr_rect (start 98.3 43.05) (end 147.5 151.15) (stroke (width 0.1) (type default)) (fill none) (layer "Edge.Cuts"))
 (segment (start 144.5 139.6925) (end 144.5 118.55) (width 1) (layer "F.Cu") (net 3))
 (segment (start 144.5 118.55) (end 134.79 108.84) (width 1) (layer "F.Cu") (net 3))
 (segment (start 140.1675 141.9) (end 142.2925 141.9) (width 1) (layer "F.Cu") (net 3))
 (segment (start 134.79 108.84) (end 132.41 108.84) (width 1) (layer "F.Cu") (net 3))
 (segment (start 142.2925 141.9) (end 144.5 139.6925) (width 1) (layer "F.Cu") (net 3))
 (segment (start 132.41 108.84) (end 133.612081 108.84) (width 1) (layer "F.Cu") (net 3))
 (segment (start 105.61 139.74) (end 106.812081 139.74) (width 1) (layer "B.Cu") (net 3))
 (segment (start 133.77 108.84) (end 132.41 108.84) (width 1) (layer "B.Cu") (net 3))
 (segment (start 108.331 81.915) (end 107.496 82.75) (width 1) (layer "B.Cu") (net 3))
 (segment (start 136.75 141.9) (end 140.1675 141.9) (width 1) (layer "B.Cu") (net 3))
 (segment (start 130.04 85.75) (end 135.3 91.01) (width 1) (layer "B.Cu") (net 3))
 (segment (start 134.42 144.23) (end 136.75 141.9) (width 1) (layer "B.Cu") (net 3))
 (segment (start 124.54 80.25) (end 108.472 80.25) (width 1) (layer "B.Cu") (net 3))
 (segment (start 113.4425 47.0575) (end 115.57 47.0575) (width 1) (layer "B.Cu") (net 3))
 (segment (start 107.496 82.75) (end 105.5 82.75) (width 1) (layer "B.Cu") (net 3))
 (segment (start 105.5 71.29) (end 108.331 74.121) (width 1) (layer "B.Cu") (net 3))
 (segment (start 112 64.79) (end 112 48.5) (width 1) (layer "B.Cu") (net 3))
 (segment (start 112 48.5) (end 113.4425 47.0575) (width 1) (layer "B.Cu") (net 3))
 (segment (start 135.3 107.31) (end 133.77 108.84) (width 1) (layer "B.Cu") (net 3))
 (segment (start 105.5 71.29) (end 112 64.79) (width 1) (layer "B.Cu") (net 3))
 (segment (start 107 140) (end 111.23 144.23) (width 1) (layer "B.Cu") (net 3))
 (segment (start 101.6 71.29) (end 101.27 70.96) (width 1) (layer "B.Cu") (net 3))
 (segment (start 108.472 80.25) (end 108.331 80.391) (width 1) (layer "B.Cu") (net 3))
 (segment (start 106.812081 139.74) (end 107 139.927919) (width 1) (layer "B.Cu") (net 3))
 (segment (start 130.04 85.75) (end 124.54 80.25) (width 1) (layer "B.Cu") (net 3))
 (segment (start 105.5 71.29) (end 101.6 71.29) (width 1) (layer "B.Cu") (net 3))
 (segment (start 135.3 91.01) (end 135.3 107.31) (width 1) (layer "B.Cu") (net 3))
 (segment (start 111.23 144.23) (end 134.42 144.23) (width 1) (layer "B.Cu") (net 3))
 (segment (start 107 139.927919) (end 107 140) (width 1) (layer "B.Cu") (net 3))
 (segment (start 108.331 74.121) (end 108.331 80.391) (width 1) (layer "B.Cu") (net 3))
 (segment (start 108.331 80.391) (end 108.331 81.915) (width 1) (layer "B.Cu") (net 3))
 (segment (start 103.17 84.62) (end 103.17 82.677) (width 1) (layer "F.Cu") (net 1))
 (segment (start 138.43 97.282) (end 138.43 89.916) (width 1.4) (layer "F.Cu") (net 1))
 (segment (start 132.41 103.759) (end 132.41 106.3) (width 1) (layer "F.Cu") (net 1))
 (segment (start 105.61 99.1) (end 102.45 99.1) (width 1) (layer "F.Cu") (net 1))
 (segment (start 101.1 97.75) (end 101.1 86.69) (width 1) (layer "F.Cu") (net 1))
 (segment (start 108.75 59.75) (end 103.42 65.08) (width 1) (layer "F.Cu") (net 1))
 (segment (start 132.41 95.75) (end 132.47104 95.68896) (width 1) (layer "F.Cu") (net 1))
 (segment (start 129.39 137.2) (end 123.39 137.2) (width 1) (layer "F.Cu") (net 1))
 (segment (start 105.5 80.25) (end 103.537 80.25) (width 1.4) (layer "F.Cu") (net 1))
 (segment (start 127.5 85.75) (end 129.75 83.5) (width 1) (layer "F.Cu") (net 1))
 (segment (start 101.92 73.75) (end 103.17 72.5) (width 1) (layer "F.Cu") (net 1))
 (segment (start 137.95 83.5) (end 140.2 85.75) (width 1) (layer "F.Cu") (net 1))
 (segment (start 106.92 80.25) (end 105.5 80.25) (width 1) (layer "F.Cu") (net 1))
 (segment (start 108.75 55.305) (end 108.75 59.75) (width 1) (layer "F.Cu") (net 1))
 (segment (start 103.42 72.25) (end 103.17 72.5) (width 1) (layer "F.Cu") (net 1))
 (segment (start 107.5 54.055) (end 108.75 55.305) (width 1) (layer "F.Cu") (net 1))
 (segment (start 130.65 138.46) (end 130.86 138.25) (width 1) (layer "F.Cu") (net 1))
 (segment (start 103.17 82.677) (end 103.17 79.883) (width 1) (layer "F.Cu") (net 1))
 (segment (start 103.17 82.677) (end 103.243 82.75) (width 1) (layer "F.Cu") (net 1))
 (segment (start 132.47104 95.508858) (end 140.25 87.729898) (width 1) (layer "F.Cu") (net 1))
 (segment (start 123.538 81.788) (end 108.458 81.788) (width 1) (layer "F.Cu") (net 1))
 (segment (start 127.5 85.75) (end 123.538 81.788) (width 1) (layer "F.Cu") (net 1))
 (segment (start 138.15 134.4) (end 140.1675 134.4) (width 1) (layer "F.Cu") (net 1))
 (segment (start 101.1 86.69) (end 103.17 84.62) (width 1) (layer "F.Cu") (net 1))
 (segment (start 140.25 87.25) (end 140.2 87.2) (width 1) (layer "F.Cu") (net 1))
 (segment (start 103.42 65.08) (end 103.42 72.25) (width 1) (layer "F.Cu") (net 1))
 (segment (start 140.2 87.2) (end 140.2 85.75) (width 1) (layer "F.Cu") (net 1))
 (segment (start 140.25 87.729898) (end 140.25 87.25) (width 1) (layer "F.Cu") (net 1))
 (segment (start 103.537 80.25) (end 103.17 79.883) (width 1.4) (layer "F.Cu") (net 1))
 (segment (start 138.43 97.282) (end 138.43 98.171) (width 1) (layer "F.Cu") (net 1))
 (segment (start 132.842 103.759) (end 132.41 103.759) (width 1) (layer "F.Cu") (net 1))
 (segment (start 102.45 99.1) (end 101.1 97.75) (width 1) (layer "F.Cu") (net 1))
 (segment (start 130.86 138.25) (end 134.3 138.25) (width 1) (layer "F.Cu") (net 1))
 (segment (start 108.458 81.788) (end 106.92 80.25) (width 1) (layer "F.Cu") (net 1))
 (segment (start 132.47104 95.68896) (end 132.47104 95.508858) (width 1) (layer "F.Cu") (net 1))
 (segment (start 123.39 99.1) (end 129.06 99.1) (width 1) (layer "F.Cu") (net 1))
 (segment (start 138.43 98.171) (end 132.842 103.759) (width 1) (layer "F.Cu") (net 1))
 (segment (start 138.43 89.916) (end 138.246949 89.732949) (width 1.4) (layer "F.Cu") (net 1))
 (segment (start 103.17 79.883) (end 103.17 72.5) (width 1) (layer "F.Cu") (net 1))
 (segment (start 129.06 99.1) (end 132.47104 95.68896) (width 1) (layer "F.Cu") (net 1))
 (segment (start 130.65 138.46) (end 129.39 137.2) (width 1) (layer "F.Cu") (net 1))
 (segment (start 129.75 83.5) (end 137.95 83.5) (width 1) (layer "F.Cu") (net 1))
 (segment (start 134.3 138.25) (end 138.15 134.4) (width 1) (layer "F.Cu") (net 1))
 (segment (start 101.52 73.75) (end 101.92 73.75) (width 1) (layer "F.Cu") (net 1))
 (segment (start 140.2 85.75) (end 142.74 85.75) (width 1) (layer "B.Cu") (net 1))
 (segment (start 132.41 111.38) (end 132.192283 111.38) (width 1) (layer "F.Cu") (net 4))
 (segment (start 127.532283 106.72) (end 123.39 106.72) (width 1) (layer "F.Cu") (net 4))
 (segment (start 132.192283 111.38) (end 127.532283 106.72) (width 1) (layer "F.Cu") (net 4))
 (segment (start 131.207919 113.92) (end 126.547919 109.26) (width 1) (layer "F.Cu") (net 5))
 (segment (start 126.547919 109.26) (end 123.39 109.26) (width 1) (layer "F.Cu") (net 5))
 (segment (start 132.41 113.92) (end 131.207919 113.92) (width 1) (layer "F.Cu") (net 5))
 (segment (start 112.56 89.93) (end 108.76 86.13) (width 1) (layer "F.Cu") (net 33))
 (segment (start 119.44 89.93) (end 112.56 89.93) (width 1) (layer "F.Cu") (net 33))
 (segment (start 119.44 89.93) (end 119.44 119.492081) (width 1) (layer "B.Cu") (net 33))
 (segment (start 119.44 119.492081) (end 106.812081 132.12) (width 1) (layer "B.Cu") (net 33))
 (segment (start 106.812081 132.12) (end 105.61 132.12) (width 1) (layer "B.Cu") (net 33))
 (segment (start 123.39 142.28) (end 123.605 142.495) (width 1) (layer "F.Cu") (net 8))
 (segment (start 123.605 139.955) (end 123.39 139.74) (width 1) (layer "F.Cu") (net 9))
 (segment (start 133.43 97.282) (end 133.43 97.71) (width 1.4) (layer "F.Cu") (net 2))
 (segment (start 133.43 97.71) (end 126.96 104.18) (width 1.4) (layer "F.Cu") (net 2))
 (segment (start 126.96 104.18) (end 123.39 104.18) (width 1.4) (layer "F.Cu") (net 2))
 (segment (start 100.5 54.75) (end 99.17 56.08) (width 1) (layer "B.Cu") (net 51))
 (segment (start 99.17 56.08) (end 99.17 75.94) (width 1) (layer "B.Cu") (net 51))
 (segment (start 99.52 76.29) (end 101.52 76.29) (width 1) (layer "B.Cu") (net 51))
 (segment (start 99.17 75.94) (end 99.52 76.29) (width 1) (layer "B.Cu") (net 51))
 (segment (start 129.573312 127.04) (end 139.433312 136.9) (width 1) (layer "B.Cu") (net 6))
 (segment (start 123.39 127.04) (end 129.573312 127.04) (width 1) (layer "B.Cu") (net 6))
 (segment (start 139.433312 136.9) (end 140.1675 136.9) (width 1) (layer "B.Cu") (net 6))
 (segment (start 140.1675 139.4) (end 136.704416 139.4) (width 1) (layer "B.Cu") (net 7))
 (segment (start 127.9 138.95) (end 127.9 130.95) (width 1) (layer "B.Cu") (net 7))
 (segment (start 136.704416 139.4) (end 134.754416 141.35) (width 1) (layer "B.Cu") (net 7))
 (segment (start 130.3 141.35) (end 127.9 138.95) (width 1) (layer "B.Cu") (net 7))
 (segment (start 126.53 129.58) (end 123.39 129.58) (width 1) (layer "B.Cu") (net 7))
 (segment (start 127.9 130.95) (end 126.53 129.58) (width 1) (layer "B.Cu") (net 7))
 (segment (start 134.754416 141.35) (end 130.3 141.35) (width 1) (layer "B.Cu") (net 7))
 (segment (start 101.99 101.64) (end 101.5 101.15) (width 1) (layer "B.Cu") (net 22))
 (segment (start 100.991 85.25) (end 99.5 86.741) (width 1.4) (layer "B.Cu") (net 22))
 (segment (start 101.5 101.15) (end 101.5 101.55) (width 1) (layer "B.Cu") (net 22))
 (segment (start 99.5 99.15) (end 101.5 101.15) (width 1) (layer "B.Cu") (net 22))
 (segment (start 105.5 85.25) (end 100.991 85.25) (width 1.4) (layer "B.Cu") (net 22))
 (segment (start 99.5 86.741) (end 99.5 99.15) (width 1) (layer "B.Cu") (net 22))
 (segment (start 105.61 101.64) (end 101.99 101.64) (width 1) (layer "B.Cu") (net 22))
 (segment (start 110.1 97.15) (end 118.1 97.15) (width 1) (layer "F.Cu") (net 20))
 (segment (start 124.12 89.93) (end 129.6 89.93) (width 1) (layer "F.Cu") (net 20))
 (segment (start 121.44 92.61) (end 124.12 89.93) (width 1) (layer "F.Cu") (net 20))
 (segment (start 135.07 89.93) (end 137.66 87.34) (width 1) (layer "F.Cu") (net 20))
 (segment (start 118.1 97.15) (end 121.44 93.81) (width 1) (layer "F.Cu") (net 20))
 (segment (start 121.44 93.81) (end 121.44 92.61) (width 1) (layer "F.Cu") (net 20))
 (segment (start 129.6 89.93) (end 135.07 89.93) (width 1) (layer "F.Cu") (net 20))
 (segment (start 106.97 94.02) (end 110.1 97.15) (width 1) (layer "F.Cu") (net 20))
 (segment (start 137.66 87.34) (end 137.66 85.75) (width 1) (layer "F.Cu") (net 20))
 (segment (start 105.61 94.02) (end 106.97 94.02) (width 1) (layer "F.Cu") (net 20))
 (segment (start 129.6 89.93) (end 129.9 89.63) (width 1) (layer "F.Cu") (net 20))
 (segment (start 137.52 85.73) (end 137.52 85.947717) (width 1) (layer "B.Cu") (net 20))
 (segment (start 135.12 85.75) (end 135.12 86.952081) (width 1) (layer "F.Cu") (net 21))
 (segment (start 120.83 88) (end 119.08 86.25) (width 1) (layer "F.Cu") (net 21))
 (segment (start 134.072081 88) (end 120.83 88) (width 1) (layer "F.Cu") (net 21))
 (segment (start 135.12 86.952081) (end 134.072081 88) (width 1) (layer "F.Cu") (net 21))
 (segment (start 105.61 96.56) (end 105.827717 96.56) (width 1) (layer "B.Cu") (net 21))
 (segment (start 114.25 86.25) (end 119.08 86.25) (width 1) (layer "B.Cu") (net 21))
 (segment (start 105.61 96.56) (end 109.75 92.42) (width 1) (layer "B.Cu") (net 21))
 (segment (start 109.75 90.75) (end 114.25 86.25) (width 1) (layer "B.Cu") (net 21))
 (segment (start 109.75 92.42) (end 109.75 90.75) (width 1) (layer "B.Cu") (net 21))
 (segment (start 102.41 52.21) (end 106.75 56.55) (width 1) (layer "F.Cu") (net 50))
 (segment (start 100.5 52.21) (end 102.41 52.21) (width 1) (layer "F.Cu") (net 50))
 (segment (start 106.75 56.55) (end 106.75 57) (width 1) (layer "F.Cu") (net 50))
 (segment (start 135.806 72.056) (end 145.5 81.75) (width 1) (layer "B.Cu") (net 14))
 (segment (start 137.03 59.7575) (end 135.806 60.9815) (width 1) (layer "B.Cu") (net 14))
 (segment (start 135.806 60.9815) (end 135.806 72.056) (width 1) (layer "B.Cu") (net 14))
 (segment (start 129.667717 119.42) (end 123.39 119.42) (width 1) (layer "B.Cu") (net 14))
 (segment (start 145.5 103.587717) (end 142.932 106.155717) (width 1) (layer "B.Cu") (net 14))
 (segment (start 145.5 81.75) (end 145.5 103.587717) (width 1) (layer "B.Cu") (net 14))
 (segment (start 142.932 106.155717) (end 129.667717 119.42) (width 1) (layer "B.Cu") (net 14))
 (segment (start 138.43 59.7575) (end 137.03 59.7575) (width 1) (layer "B.Cu") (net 14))
 (segment (start 111.6525 49.5975) (end 107.5 45.445) (width 1) (layer "F.Cu") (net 43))
 (segment (start 115.57 49.5975) (end 111.6525 49.5975) (width 1) (layer "F.Cu") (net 43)))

